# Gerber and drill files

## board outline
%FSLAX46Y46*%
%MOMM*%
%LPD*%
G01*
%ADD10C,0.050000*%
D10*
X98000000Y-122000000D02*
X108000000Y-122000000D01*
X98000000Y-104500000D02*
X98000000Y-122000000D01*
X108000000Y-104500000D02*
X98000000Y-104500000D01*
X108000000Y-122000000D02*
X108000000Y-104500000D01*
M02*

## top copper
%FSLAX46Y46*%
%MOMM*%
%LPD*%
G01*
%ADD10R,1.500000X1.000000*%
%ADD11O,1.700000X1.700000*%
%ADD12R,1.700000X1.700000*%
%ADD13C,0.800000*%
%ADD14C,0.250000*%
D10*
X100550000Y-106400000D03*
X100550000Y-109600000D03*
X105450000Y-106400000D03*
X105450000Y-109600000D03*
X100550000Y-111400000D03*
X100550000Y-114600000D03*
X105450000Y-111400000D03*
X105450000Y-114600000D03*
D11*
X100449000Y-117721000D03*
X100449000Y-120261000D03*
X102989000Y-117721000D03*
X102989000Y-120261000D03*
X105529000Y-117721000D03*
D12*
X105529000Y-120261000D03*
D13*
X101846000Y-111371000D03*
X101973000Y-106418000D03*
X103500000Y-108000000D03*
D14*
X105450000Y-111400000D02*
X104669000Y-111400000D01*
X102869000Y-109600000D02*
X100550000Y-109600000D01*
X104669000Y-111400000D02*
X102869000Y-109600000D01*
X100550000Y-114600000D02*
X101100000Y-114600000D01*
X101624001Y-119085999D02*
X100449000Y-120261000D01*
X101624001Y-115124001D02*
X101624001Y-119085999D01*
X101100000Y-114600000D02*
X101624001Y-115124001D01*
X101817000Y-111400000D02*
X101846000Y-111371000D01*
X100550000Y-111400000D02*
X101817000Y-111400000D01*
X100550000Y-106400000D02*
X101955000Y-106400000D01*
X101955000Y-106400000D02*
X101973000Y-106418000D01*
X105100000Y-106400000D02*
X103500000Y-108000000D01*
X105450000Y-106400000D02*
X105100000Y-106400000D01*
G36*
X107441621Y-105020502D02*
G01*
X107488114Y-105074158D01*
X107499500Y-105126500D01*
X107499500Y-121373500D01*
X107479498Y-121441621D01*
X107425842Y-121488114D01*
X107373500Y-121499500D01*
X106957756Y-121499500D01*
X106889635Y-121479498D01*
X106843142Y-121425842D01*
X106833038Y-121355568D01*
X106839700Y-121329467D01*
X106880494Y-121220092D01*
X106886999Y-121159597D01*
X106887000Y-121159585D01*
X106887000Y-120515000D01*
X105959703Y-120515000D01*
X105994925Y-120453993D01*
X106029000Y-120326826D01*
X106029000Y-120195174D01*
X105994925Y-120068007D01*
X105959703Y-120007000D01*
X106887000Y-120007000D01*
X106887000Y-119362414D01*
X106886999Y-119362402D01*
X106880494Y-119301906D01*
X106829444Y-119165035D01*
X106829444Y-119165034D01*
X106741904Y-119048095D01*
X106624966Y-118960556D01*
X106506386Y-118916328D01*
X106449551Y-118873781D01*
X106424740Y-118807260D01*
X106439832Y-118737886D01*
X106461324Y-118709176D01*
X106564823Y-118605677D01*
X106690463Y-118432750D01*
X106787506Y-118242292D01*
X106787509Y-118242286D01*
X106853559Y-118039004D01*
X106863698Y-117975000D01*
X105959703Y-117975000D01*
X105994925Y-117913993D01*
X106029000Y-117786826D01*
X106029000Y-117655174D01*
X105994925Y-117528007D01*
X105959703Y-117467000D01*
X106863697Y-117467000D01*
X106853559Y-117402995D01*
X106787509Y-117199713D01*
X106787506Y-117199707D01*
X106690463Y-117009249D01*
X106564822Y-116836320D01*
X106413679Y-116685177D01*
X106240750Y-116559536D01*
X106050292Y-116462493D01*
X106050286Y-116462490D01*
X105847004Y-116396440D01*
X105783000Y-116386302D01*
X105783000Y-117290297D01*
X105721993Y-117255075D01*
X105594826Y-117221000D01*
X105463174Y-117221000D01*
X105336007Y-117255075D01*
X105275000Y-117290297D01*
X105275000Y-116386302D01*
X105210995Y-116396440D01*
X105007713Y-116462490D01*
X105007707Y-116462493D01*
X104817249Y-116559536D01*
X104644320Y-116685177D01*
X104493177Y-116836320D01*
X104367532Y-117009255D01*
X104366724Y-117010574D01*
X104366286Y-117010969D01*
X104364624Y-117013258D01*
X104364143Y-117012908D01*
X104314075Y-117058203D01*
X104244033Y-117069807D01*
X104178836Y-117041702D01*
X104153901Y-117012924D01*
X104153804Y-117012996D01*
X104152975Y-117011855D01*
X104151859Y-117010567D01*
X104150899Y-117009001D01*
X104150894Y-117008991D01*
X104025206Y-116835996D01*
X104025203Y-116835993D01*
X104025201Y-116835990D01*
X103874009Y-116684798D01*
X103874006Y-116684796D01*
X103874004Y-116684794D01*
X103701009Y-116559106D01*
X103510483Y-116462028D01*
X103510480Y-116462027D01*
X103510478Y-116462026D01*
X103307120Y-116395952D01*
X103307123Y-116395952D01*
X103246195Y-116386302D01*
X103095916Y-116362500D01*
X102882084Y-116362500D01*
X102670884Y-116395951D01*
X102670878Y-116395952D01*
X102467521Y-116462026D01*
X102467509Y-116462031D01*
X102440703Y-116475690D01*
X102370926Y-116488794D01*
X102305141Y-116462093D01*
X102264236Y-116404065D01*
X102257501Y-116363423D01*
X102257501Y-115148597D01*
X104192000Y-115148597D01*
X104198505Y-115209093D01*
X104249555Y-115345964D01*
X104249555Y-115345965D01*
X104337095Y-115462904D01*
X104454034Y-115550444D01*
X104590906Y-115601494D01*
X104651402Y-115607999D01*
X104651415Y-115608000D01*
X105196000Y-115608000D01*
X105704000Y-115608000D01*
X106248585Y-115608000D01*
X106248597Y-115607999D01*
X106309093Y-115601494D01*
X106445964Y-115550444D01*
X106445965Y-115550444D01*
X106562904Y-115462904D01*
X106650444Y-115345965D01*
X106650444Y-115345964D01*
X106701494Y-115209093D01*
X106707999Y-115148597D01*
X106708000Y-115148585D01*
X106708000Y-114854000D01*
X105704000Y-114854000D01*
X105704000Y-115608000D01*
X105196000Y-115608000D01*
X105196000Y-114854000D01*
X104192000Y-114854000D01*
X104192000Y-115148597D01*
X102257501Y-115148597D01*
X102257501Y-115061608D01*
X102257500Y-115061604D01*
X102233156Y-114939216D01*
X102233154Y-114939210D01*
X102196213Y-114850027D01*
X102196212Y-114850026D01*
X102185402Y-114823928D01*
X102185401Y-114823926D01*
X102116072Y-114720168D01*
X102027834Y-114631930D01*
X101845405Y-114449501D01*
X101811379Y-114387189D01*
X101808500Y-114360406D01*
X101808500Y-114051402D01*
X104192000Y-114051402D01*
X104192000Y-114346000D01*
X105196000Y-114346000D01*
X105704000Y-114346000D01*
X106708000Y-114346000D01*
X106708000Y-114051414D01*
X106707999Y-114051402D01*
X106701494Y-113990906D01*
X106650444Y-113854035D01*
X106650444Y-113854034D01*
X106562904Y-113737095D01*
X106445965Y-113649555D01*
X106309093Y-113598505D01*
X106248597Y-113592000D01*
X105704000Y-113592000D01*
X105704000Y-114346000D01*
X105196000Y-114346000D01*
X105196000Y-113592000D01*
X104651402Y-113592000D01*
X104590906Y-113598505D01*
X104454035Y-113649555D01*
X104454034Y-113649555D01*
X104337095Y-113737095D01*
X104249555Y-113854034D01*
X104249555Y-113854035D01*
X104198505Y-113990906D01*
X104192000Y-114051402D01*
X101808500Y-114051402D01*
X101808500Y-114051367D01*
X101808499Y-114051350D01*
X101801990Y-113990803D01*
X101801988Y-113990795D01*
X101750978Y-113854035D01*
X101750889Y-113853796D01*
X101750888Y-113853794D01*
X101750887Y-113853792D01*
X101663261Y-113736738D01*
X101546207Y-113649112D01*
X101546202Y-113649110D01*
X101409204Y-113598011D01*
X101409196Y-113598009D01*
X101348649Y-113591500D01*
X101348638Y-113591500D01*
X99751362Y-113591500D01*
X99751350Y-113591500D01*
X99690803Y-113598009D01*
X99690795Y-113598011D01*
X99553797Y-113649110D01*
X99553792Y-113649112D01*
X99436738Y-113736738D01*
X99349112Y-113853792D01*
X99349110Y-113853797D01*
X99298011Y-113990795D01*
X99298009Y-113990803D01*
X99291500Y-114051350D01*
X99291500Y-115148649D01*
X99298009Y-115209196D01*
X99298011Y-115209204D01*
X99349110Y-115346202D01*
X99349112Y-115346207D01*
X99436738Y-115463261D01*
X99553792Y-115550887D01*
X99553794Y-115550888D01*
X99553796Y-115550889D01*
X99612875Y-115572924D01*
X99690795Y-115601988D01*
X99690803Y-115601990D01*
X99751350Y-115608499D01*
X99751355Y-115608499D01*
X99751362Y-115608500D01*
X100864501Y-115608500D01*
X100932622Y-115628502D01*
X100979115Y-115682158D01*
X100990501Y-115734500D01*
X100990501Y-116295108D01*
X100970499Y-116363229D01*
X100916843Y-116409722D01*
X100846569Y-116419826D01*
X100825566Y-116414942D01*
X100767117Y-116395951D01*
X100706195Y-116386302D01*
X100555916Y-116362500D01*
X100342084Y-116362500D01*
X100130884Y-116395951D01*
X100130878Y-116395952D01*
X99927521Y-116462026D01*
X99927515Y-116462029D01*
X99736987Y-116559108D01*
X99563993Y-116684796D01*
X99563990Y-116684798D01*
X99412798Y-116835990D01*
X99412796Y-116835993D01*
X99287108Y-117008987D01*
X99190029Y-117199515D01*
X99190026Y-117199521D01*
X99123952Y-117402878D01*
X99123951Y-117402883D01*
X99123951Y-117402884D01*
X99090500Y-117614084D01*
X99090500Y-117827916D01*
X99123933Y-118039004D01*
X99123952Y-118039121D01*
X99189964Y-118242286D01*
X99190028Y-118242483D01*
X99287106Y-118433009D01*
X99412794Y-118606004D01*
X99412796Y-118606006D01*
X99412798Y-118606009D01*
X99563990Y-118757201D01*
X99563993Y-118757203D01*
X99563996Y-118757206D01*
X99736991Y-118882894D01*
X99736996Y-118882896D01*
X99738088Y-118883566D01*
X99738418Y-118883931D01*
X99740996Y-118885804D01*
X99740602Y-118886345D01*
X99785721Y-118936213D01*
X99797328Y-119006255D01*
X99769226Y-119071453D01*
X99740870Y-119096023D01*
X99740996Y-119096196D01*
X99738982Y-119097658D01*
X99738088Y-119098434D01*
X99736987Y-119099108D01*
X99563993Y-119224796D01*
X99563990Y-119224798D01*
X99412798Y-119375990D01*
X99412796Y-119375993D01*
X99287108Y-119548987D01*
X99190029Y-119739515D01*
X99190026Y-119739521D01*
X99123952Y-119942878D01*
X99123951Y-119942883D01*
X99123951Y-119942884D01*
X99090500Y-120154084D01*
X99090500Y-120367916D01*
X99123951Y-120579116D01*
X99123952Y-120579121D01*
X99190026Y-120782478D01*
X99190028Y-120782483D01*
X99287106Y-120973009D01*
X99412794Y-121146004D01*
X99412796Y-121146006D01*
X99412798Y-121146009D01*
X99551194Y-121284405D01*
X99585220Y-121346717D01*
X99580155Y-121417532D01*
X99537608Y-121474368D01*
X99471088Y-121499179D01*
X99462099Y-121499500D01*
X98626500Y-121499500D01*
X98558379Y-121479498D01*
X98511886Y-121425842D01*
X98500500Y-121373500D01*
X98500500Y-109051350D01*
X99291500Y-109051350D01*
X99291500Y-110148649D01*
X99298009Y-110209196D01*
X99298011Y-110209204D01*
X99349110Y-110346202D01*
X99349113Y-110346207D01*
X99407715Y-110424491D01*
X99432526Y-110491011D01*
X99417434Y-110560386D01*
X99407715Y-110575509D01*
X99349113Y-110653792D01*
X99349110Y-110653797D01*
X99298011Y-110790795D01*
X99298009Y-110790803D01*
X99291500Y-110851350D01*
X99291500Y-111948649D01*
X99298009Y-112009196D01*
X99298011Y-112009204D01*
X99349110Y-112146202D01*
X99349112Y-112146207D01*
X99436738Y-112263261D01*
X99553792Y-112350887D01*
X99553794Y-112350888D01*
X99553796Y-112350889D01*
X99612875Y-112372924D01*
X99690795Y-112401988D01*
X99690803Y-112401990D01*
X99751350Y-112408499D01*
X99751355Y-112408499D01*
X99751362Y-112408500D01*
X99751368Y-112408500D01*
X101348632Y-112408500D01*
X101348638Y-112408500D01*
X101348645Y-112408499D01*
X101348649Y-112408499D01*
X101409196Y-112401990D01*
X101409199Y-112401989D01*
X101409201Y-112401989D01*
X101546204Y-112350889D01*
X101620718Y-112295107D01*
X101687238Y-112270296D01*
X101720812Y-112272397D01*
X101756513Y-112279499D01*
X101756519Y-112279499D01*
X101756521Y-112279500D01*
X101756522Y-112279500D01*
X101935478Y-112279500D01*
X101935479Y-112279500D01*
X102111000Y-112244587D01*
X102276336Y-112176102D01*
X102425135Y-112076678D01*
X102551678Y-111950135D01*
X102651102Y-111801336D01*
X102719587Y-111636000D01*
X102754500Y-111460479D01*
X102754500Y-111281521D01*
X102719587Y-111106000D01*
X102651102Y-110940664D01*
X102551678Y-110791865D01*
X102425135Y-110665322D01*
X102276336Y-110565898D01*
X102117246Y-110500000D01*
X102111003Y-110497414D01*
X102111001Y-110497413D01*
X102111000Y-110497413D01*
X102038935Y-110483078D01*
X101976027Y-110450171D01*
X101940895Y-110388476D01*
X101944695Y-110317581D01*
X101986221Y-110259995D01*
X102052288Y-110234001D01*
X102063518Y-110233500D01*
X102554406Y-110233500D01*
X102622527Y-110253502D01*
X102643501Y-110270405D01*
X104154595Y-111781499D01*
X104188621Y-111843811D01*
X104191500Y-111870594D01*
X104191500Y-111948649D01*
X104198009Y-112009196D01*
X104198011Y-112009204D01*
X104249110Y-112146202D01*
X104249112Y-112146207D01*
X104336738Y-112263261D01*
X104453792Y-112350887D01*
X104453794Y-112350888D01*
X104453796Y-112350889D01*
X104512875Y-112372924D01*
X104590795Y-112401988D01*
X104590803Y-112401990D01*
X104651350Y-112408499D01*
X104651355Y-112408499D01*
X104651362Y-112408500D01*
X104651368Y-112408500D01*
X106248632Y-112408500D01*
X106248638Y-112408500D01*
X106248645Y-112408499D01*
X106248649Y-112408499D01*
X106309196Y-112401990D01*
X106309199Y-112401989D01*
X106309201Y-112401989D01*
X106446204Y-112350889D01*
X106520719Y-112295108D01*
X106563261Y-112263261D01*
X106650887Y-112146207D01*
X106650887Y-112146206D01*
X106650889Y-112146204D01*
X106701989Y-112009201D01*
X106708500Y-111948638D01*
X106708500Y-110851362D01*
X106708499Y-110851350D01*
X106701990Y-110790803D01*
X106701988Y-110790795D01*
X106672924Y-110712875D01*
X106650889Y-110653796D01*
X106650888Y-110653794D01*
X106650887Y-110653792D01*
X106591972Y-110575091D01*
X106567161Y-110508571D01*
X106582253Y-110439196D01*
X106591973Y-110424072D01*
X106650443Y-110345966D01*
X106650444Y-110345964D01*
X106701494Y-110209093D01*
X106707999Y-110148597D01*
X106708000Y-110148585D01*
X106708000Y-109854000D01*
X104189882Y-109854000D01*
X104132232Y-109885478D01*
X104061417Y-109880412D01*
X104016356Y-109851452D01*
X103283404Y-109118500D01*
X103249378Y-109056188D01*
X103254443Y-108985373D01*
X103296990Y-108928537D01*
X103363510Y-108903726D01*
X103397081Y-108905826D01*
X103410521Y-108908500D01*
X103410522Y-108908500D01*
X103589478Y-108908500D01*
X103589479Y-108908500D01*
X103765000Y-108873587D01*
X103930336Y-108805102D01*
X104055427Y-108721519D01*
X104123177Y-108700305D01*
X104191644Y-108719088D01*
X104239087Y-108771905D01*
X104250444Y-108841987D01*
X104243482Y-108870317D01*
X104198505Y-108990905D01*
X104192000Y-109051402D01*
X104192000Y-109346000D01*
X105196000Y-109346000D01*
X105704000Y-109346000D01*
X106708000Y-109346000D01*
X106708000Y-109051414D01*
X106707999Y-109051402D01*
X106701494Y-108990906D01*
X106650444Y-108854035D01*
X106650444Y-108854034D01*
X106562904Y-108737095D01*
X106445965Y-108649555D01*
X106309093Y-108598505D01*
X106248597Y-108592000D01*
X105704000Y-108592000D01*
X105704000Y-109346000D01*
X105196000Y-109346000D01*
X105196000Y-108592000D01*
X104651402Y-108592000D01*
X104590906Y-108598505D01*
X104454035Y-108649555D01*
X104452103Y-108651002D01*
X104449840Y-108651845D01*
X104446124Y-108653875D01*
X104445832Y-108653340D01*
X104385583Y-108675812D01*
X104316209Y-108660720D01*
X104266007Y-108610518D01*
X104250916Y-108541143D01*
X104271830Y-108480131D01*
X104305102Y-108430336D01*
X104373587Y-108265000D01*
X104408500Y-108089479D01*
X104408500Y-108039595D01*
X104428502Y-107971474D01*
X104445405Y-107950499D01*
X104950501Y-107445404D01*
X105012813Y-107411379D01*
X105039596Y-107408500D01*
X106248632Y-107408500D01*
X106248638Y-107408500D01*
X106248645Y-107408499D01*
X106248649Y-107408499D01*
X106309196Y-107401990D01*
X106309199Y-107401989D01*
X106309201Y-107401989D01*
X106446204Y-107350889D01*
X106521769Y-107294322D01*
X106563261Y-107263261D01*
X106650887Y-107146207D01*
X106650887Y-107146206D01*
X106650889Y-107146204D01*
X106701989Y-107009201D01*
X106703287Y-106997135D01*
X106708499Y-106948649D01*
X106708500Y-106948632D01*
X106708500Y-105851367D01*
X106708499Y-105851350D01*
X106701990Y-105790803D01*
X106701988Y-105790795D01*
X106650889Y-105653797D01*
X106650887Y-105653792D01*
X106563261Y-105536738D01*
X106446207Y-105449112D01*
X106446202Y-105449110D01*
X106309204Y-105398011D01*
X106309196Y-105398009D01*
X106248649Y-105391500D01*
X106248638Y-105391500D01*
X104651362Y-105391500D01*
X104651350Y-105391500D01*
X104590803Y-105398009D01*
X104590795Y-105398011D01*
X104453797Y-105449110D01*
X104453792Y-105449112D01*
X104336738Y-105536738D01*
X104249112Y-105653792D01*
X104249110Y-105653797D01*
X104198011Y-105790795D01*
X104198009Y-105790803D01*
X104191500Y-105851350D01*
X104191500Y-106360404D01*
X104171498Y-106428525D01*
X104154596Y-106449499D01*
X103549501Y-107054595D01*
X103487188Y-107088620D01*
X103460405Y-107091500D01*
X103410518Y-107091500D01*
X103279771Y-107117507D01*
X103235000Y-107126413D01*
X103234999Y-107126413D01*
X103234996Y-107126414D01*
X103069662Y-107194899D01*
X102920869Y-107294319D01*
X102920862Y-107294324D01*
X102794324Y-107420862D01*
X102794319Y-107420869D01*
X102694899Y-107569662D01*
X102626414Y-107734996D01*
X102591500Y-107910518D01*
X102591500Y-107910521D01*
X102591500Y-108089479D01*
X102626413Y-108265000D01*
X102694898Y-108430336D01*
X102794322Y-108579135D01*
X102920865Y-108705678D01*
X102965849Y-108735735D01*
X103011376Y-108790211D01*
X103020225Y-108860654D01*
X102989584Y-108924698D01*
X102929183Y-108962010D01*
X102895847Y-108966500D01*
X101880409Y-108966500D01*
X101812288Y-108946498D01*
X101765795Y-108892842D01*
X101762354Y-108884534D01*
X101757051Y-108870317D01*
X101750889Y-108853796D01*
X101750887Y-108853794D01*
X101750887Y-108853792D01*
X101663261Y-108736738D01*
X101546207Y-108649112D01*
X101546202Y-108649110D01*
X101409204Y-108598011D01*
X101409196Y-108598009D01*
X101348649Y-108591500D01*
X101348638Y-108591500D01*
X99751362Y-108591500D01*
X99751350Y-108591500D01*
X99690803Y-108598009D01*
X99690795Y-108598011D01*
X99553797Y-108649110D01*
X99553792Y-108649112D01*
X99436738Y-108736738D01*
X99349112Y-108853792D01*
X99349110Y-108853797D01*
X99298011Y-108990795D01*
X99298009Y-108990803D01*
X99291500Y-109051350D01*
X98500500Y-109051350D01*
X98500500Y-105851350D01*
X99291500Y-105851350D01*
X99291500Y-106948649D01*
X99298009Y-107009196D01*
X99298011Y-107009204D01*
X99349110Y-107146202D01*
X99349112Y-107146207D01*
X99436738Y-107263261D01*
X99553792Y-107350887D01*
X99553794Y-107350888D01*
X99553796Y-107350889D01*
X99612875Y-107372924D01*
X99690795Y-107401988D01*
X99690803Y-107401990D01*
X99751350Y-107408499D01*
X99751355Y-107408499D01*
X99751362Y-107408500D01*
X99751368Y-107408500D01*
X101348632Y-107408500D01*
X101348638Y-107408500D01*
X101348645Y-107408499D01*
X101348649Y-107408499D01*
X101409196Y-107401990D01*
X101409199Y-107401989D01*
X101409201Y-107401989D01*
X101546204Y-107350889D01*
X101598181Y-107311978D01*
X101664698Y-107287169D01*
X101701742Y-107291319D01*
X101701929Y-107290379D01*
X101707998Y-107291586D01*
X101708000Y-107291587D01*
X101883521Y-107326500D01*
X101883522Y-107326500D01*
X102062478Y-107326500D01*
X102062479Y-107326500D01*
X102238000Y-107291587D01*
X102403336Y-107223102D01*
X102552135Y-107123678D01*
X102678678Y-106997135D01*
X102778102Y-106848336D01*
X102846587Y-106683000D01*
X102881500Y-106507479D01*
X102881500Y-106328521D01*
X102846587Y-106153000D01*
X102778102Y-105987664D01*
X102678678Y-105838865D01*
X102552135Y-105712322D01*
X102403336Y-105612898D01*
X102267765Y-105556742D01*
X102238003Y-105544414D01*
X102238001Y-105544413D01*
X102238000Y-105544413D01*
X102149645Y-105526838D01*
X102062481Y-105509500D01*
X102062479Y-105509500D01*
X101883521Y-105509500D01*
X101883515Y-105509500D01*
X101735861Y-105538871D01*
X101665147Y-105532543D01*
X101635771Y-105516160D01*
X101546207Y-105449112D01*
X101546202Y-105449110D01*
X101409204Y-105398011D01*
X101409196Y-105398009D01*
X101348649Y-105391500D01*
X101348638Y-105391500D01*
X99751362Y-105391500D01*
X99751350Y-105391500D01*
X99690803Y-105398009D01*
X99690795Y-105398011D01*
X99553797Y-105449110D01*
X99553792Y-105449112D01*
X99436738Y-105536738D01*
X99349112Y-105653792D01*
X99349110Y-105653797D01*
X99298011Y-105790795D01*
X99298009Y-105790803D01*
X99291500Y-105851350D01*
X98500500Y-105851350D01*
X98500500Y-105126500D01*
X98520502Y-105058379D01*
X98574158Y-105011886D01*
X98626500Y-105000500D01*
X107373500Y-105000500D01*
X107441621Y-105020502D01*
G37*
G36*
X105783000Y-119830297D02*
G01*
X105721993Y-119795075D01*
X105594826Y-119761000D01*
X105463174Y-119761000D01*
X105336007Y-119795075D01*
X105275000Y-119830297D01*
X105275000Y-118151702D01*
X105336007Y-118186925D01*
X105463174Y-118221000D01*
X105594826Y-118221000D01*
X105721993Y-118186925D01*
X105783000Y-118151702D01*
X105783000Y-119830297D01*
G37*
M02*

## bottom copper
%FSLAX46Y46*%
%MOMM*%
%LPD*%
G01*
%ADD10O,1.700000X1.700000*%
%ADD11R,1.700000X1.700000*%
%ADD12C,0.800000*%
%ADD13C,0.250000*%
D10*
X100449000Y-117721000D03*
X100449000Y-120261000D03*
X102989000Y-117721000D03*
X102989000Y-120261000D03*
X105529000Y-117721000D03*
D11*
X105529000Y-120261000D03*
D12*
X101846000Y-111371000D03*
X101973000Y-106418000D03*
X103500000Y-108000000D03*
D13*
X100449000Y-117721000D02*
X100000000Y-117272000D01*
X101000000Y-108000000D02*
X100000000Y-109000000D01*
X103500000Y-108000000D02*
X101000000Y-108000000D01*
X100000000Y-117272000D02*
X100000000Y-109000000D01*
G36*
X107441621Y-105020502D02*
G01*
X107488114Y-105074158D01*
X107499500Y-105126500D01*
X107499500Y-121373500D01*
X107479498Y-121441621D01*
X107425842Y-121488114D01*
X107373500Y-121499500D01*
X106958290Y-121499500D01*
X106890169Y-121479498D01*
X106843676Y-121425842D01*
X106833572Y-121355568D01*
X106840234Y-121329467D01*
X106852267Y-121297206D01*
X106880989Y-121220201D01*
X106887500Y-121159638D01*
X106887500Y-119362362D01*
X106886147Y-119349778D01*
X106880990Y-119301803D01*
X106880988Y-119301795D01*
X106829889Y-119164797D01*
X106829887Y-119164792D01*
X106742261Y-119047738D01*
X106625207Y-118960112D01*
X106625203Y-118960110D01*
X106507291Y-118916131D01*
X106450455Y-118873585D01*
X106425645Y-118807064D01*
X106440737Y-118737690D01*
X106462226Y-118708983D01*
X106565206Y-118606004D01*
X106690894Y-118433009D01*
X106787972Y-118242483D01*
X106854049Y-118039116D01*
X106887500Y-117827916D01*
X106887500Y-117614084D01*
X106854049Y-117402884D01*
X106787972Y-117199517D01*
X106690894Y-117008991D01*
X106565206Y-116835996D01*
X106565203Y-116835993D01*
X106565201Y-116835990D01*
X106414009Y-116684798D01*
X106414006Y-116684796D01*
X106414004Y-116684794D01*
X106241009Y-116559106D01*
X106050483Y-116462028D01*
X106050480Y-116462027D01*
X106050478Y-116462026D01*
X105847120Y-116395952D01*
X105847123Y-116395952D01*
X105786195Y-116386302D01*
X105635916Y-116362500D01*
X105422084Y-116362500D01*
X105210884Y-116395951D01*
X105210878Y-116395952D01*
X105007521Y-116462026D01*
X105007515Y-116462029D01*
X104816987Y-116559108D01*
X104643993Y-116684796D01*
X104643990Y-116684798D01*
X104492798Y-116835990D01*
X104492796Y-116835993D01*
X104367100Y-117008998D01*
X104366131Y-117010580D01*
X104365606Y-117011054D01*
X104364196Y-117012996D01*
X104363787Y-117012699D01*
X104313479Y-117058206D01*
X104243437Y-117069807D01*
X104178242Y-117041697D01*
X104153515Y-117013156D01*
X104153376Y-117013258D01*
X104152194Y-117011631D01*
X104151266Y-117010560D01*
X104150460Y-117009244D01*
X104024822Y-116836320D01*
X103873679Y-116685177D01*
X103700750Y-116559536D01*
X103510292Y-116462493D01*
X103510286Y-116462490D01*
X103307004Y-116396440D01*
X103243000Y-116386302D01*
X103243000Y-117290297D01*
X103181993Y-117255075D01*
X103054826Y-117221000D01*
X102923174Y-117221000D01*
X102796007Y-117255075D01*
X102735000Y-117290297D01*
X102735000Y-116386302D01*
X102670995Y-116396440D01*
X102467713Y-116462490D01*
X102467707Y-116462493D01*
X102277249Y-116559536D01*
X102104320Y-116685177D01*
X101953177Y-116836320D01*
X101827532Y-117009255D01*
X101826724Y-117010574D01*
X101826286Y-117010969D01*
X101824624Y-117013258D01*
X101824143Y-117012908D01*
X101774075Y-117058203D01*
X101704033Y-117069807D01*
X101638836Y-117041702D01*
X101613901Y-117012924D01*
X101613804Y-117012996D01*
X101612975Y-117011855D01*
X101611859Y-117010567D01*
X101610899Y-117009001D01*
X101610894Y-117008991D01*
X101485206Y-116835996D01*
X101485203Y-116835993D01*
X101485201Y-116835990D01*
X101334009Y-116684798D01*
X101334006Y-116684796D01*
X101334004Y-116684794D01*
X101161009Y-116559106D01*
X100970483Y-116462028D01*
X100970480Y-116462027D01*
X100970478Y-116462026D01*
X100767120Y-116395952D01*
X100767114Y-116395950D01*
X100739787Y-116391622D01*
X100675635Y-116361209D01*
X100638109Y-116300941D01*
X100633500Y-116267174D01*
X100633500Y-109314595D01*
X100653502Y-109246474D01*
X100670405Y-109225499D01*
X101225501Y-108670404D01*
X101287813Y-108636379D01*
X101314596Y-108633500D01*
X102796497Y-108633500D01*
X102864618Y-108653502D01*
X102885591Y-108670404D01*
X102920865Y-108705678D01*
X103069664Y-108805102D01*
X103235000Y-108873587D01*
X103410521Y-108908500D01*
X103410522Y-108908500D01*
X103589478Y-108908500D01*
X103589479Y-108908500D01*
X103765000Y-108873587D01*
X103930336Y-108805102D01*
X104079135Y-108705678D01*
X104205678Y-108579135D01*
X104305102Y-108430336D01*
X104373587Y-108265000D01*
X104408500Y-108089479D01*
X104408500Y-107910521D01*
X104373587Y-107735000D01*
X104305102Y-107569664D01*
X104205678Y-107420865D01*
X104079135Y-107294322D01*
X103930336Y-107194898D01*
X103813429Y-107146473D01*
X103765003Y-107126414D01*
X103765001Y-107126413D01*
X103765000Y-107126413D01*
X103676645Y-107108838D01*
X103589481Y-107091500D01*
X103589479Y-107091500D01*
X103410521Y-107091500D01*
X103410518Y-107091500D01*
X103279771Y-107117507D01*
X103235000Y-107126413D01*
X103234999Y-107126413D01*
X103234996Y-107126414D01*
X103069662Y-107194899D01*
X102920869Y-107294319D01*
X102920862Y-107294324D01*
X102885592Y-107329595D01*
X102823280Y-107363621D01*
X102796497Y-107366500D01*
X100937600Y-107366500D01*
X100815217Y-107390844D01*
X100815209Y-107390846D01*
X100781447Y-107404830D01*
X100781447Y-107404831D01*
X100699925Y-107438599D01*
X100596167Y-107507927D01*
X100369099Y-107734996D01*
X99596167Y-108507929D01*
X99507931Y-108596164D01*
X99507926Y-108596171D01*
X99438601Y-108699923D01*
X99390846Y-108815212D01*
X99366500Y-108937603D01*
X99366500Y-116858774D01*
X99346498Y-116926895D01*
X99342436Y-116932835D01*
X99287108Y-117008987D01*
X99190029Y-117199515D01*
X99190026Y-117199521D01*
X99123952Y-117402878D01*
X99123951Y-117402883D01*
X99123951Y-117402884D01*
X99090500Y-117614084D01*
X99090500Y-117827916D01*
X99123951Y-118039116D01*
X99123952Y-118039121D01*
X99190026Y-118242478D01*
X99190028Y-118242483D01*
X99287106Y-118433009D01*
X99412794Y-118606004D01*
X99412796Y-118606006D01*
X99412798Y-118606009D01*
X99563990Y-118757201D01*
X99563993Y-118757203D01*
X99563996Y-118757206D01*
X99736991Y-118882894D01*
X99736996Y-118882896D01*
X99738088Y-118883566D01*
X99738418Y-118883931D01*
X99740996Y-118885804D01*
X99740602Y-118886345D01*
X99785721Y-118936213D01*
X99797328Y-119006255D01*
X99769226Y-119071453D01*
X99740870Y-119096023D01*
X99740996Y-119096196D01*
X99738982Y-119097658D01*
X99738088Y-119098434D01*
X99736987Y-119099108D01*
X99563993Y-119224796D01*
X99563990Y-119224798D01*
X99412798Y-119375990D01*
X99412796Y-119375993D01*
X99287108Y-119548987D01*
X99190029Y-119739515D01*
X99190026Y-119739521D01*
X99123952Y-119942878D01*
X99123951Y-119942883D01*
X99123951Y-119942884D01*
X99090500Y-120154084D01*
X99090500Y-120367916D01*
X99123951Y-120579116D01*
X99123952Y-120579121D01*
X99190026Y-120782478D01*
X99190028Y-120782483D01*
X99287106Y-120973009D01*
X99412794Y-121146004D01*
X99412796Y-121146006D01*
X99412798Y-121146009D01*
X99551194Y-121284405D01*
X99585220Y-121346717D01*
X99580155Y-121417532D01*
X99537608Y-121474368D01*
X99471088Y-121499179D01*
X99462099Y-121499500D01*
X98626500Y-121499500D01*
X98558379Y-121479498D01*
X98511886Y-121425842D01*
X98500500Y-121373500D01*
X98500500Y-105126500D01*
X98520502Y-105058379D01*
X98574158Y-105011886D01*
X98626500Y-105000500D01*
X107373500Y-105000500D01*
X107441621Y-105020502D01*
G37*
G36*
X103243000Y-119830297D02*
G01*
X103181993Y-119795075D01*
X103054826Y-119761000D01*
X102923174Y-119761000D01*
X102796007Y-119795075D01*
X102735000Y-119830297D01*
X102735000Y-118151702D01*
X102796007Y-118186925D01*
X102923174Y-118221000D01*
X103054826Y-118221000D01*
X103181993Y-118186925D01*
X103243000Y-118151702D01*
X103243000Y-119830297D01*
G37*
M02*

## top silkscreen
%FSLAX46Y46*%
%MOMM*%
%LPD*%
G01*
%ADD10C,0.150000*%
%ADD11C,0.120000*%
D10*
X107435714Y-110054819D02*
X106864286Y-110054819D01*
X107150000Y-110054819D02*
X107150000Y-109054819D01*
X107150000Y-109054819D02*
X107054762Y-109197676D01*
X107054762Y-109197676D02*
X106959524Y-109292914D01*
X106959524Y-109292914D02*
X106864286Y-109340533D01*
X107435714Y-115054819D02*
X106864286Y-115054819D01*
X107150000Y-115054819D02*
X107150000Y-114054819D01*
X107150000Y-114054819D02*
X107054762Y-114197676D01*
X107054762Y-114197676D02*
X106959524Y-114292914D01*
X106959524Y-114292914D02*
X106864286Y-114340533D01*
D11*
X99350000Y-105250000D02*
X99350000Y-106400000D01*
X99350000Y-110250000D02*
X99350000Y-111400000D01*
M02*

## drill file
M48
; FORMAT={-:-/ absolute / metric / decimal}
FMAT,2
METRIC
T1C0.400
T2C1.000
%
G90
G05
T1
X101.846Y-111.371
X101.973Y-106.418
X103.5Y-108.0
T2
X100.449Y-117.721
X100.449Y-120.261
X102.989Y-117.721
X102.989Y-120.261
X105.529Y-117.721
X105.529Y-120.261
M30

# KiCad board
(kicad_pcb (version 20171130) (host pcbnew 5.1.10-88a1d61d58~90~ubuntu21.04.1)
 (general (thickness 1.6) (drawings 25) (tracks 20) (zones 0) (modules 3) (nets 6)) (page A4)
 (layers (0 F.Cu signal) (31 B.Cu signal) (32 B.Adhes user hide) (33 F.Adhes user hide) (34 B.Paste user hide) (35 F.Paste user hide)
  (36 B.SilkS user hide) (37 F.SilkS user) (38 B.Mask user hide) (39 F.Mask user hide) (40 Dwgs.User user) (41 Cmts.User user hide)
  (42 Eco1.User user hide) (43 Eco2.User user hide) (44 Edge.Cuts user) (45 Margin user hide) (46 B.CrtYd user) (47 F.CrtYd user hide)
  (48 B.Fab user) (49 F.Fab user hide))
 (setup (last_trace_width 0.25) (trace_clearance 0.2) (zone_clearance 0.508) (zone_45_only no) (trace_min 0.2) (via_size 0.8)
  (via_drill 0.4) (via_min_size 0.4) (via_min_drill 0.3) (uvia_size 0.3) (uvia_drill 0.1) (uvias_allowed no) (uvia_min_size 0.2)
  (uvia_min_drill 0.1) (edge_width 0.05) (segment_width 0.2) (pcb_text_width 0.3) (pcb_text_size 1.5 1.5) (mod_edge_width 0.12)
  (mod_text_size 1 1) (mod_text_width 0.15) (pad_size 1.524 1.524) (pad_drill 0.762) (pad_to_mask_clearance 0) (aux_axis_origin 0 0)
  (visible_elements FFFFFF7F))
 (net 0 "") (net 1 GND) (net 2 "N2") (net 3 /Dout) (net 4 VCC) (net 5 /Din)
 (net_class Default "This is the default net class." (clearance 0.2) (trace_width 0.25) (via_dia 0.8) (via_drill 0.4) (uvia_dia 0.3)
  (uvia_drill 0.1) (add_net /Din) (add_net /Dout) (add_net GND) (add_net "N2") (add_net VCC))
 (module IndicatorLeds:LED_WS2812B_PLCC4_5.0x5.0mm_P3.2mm (layer F.Cu) (at 103 108 180)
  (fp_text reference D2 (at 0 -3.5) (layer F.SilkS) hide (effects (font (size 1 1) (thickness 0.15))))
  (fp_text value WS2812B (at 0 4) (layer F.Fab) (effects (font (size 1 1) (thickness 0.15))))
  (fp_line (start 3.65 2.75) (end 3.65 1.6) (layer F.SilkS) (width 0.12))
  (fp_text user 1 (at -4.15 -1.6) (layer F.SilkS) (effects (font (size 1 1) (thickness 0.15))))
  (pad 3 smd rect (at 2.45 1.6 180) (size 1.5 1) (layers F.Cu F.Paste F.Mask) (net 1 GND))
  (pad 4 smd rect (at 2.45 -1.6 180) (size 1.5 1) (layers F.Cu F.Paste F.Mask) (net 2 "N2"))
  (pad 2 smd rect (at -2.45 1.6 180) (size 1.5 1) (layers F.Cu F.Paste F.Mask) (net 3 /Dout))
  (pad 1 smd rect (at -2.45 -1.6 180) (size 1.5 1) (layers F.Cu F.Paste F.Mask) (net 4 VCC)))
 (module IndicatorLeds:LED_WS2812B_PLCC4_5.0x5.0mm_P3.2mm (layer F.Cu) (at 103 113 180)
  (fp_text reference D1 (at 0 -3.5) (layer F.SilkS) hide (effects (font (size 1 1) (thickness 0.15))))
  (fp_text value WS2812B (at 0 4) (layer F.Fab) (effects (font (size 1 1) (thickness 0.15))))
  (fp_line (start 3.65 2.75) (end 3.65 1.6) (layer F.SilkS) (width 0.12))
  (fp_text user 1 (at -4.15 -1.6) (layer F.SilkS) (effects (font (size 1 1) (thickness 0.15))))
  (pad 3 smd rect (at 2.45 1.6 180) (size 1.5 1) (layers F.Cu F.Paste F.Mask) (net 1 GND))
  (pad 4 smd rect (at 2.45 -1.6 180) (size 1.5 1) (layers F.Cu F.Paste F.Mask) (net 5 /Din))
  (pad 2 smd rect (at -2.45 1.6 180) (size 1.5 1) (layers F.Cu F.Paste F.Mask) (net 2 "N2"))
  (pad 1 smd rect (at -2.45 -1.6 180) (size 1.5 1) (layers F.Cu F.Paste F.Mask) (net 4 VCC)))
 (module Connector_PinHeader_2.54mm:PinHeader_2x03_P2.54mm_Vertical (layer B.Cu) (at 105.529 120.261 90)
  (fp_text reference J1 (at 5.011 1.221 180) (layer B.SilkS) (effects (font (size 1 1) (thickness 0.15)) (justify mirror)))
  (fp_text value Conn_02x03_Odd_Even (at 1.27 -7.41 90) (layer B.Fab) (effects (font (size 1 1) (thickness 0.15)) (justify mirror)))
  (pad 6 thru_hole oval (at 2.54 -5.08 90) (size 1.7 1.7) (drill 1) (layers *.Cu *.Mask) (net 3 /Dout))
  (pad 5 thru_hole oval (at 0 -5.08 90) (size 1.7 1.7) (drill 1) (layers *.Cu *.Mask) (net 5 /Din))
  (pad 4 thru_hole oval (at 2.54 -2.54 90) (size 1.7 1.7) (drill 1) (layers *.Cu *.Mask) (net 1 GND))
  (pad 3 thru_hole oval (at 0 -2.54 90) (size 1.7 1.7) (drill 1) (layers *.Cu *.Mask) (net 1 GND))
  (pad 2 thru_hole oval (at 2.54 0 90) (size 1.7 1.7) (drill 1) (layers *.Cu *.Mask) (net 4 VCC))
  (pad 1 thru_hole rect (at 0 0 90) (size 1.7 1.7) (drill 1) (layers *.Cu *.Mask) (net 4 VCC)))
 (gr_line (start 98 122) (end 108 122) (layer Edge.Cuts) (width 0.05))
 (gr_line (start 98 104.5) (end 98 122) (layer Edge.Cuts) (width 0.05))
 (gr_line (start 108 104.5) (end 98 104.5) (layer Edge.Cuts) (width 0.05))
 (gr_line (start 108 122) (end 108 104.5) (layer Edge.Cuts) (width 0.05))
 (segment (start 105.45 111.4) (end 104.669 111.4) (width 0.25) (layer F.Cu) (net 2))
 (segment (start 102.869 109.6) (end 100.55 109.6) (width 0.25) (layer F.Cu) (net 2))
 (segment (start 104.669 111.4) (end 102.869 109.6) (width 0.25) (layer F.Cu) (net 2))
 (segment (start 100.55 114.6) (end 101.1 114.6) (width 0.25) (layer F.Cu) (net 5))
 (segment (start 101.624001 119.085999) (end 100.449 120.261) (width 0.25) (layer F.Cu) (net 5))
 (segment (start 101.624001 115.124001) (end 101.624001 119.085999) (width 0.25) (layer F.Cu) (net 5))
 (segment (start 101.1 114.6) (end 101.624001 115.124001) (width 0.25) (layer F.Cu) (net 5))
 (via (at 101.846 111.371) (size 0.8) (drill 0.4) (layers F.Cu B.Cu) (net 1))
 (segment (start 101.817 111.4) (end 101.846 111.371) (width 0.25) (layer F.Cu) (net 1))
 (segment (start 100.55 111.4) (end 101.817 111.4) (width 0.25) (layer F.Cu) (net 1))
 (via (at 101.973 106.418) (size 0.8) (drill 0.4) (layers F.Cu B.Cu) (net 1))
 (segment (start 100.55 106.4) (end 101.955 106.4) (width 0.25) (layer F.Cu) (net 1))
 (segment (start 101.955 106.4) (end 101.973 106.418) (width 0.25) (layer F.Cu) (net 1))
 (segment (start 100.449 117.721) (end 100 117.272) (width 0.25) (layer B.Cu) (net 3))
 (segment (start 105.1 106.4) (end 103.5 108) (width 0.25) (layer F.Cu) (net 3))
 (via (at 103.5 108) (size 0.8) (drill 0.4) (layers F.Cu B.Cu) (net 3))
 (segment (start 105.45 106.4) (end 105.1 106.4) (width 0.25) (layer F.Cu) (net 3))
 (segment (start 101 108) (end 100 109) (width 0.25) (layer B.Cu) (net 3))
 (segment (start 103.5 108) (end 101 108) (width 0.25) (layer B.Cu) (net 3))
 (segment (start 100 117.272) (end 100 109) (width 0.25) (layer B.Cu) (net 3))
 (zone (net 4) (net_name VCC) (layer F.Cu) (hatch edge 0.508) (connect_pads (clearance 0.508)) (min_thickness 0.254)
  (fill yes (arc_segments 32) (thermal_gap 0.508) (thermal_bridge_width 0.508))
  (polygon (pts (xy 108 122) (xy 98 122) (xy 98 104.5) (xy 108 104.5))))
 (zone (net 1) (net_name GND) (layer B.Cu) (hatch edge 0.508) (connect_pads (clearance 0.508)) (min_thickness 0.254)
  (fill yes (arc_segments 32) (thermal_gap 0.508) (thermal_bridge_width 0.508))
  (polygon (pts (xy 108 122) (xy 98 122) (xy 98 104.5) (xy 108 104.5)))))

